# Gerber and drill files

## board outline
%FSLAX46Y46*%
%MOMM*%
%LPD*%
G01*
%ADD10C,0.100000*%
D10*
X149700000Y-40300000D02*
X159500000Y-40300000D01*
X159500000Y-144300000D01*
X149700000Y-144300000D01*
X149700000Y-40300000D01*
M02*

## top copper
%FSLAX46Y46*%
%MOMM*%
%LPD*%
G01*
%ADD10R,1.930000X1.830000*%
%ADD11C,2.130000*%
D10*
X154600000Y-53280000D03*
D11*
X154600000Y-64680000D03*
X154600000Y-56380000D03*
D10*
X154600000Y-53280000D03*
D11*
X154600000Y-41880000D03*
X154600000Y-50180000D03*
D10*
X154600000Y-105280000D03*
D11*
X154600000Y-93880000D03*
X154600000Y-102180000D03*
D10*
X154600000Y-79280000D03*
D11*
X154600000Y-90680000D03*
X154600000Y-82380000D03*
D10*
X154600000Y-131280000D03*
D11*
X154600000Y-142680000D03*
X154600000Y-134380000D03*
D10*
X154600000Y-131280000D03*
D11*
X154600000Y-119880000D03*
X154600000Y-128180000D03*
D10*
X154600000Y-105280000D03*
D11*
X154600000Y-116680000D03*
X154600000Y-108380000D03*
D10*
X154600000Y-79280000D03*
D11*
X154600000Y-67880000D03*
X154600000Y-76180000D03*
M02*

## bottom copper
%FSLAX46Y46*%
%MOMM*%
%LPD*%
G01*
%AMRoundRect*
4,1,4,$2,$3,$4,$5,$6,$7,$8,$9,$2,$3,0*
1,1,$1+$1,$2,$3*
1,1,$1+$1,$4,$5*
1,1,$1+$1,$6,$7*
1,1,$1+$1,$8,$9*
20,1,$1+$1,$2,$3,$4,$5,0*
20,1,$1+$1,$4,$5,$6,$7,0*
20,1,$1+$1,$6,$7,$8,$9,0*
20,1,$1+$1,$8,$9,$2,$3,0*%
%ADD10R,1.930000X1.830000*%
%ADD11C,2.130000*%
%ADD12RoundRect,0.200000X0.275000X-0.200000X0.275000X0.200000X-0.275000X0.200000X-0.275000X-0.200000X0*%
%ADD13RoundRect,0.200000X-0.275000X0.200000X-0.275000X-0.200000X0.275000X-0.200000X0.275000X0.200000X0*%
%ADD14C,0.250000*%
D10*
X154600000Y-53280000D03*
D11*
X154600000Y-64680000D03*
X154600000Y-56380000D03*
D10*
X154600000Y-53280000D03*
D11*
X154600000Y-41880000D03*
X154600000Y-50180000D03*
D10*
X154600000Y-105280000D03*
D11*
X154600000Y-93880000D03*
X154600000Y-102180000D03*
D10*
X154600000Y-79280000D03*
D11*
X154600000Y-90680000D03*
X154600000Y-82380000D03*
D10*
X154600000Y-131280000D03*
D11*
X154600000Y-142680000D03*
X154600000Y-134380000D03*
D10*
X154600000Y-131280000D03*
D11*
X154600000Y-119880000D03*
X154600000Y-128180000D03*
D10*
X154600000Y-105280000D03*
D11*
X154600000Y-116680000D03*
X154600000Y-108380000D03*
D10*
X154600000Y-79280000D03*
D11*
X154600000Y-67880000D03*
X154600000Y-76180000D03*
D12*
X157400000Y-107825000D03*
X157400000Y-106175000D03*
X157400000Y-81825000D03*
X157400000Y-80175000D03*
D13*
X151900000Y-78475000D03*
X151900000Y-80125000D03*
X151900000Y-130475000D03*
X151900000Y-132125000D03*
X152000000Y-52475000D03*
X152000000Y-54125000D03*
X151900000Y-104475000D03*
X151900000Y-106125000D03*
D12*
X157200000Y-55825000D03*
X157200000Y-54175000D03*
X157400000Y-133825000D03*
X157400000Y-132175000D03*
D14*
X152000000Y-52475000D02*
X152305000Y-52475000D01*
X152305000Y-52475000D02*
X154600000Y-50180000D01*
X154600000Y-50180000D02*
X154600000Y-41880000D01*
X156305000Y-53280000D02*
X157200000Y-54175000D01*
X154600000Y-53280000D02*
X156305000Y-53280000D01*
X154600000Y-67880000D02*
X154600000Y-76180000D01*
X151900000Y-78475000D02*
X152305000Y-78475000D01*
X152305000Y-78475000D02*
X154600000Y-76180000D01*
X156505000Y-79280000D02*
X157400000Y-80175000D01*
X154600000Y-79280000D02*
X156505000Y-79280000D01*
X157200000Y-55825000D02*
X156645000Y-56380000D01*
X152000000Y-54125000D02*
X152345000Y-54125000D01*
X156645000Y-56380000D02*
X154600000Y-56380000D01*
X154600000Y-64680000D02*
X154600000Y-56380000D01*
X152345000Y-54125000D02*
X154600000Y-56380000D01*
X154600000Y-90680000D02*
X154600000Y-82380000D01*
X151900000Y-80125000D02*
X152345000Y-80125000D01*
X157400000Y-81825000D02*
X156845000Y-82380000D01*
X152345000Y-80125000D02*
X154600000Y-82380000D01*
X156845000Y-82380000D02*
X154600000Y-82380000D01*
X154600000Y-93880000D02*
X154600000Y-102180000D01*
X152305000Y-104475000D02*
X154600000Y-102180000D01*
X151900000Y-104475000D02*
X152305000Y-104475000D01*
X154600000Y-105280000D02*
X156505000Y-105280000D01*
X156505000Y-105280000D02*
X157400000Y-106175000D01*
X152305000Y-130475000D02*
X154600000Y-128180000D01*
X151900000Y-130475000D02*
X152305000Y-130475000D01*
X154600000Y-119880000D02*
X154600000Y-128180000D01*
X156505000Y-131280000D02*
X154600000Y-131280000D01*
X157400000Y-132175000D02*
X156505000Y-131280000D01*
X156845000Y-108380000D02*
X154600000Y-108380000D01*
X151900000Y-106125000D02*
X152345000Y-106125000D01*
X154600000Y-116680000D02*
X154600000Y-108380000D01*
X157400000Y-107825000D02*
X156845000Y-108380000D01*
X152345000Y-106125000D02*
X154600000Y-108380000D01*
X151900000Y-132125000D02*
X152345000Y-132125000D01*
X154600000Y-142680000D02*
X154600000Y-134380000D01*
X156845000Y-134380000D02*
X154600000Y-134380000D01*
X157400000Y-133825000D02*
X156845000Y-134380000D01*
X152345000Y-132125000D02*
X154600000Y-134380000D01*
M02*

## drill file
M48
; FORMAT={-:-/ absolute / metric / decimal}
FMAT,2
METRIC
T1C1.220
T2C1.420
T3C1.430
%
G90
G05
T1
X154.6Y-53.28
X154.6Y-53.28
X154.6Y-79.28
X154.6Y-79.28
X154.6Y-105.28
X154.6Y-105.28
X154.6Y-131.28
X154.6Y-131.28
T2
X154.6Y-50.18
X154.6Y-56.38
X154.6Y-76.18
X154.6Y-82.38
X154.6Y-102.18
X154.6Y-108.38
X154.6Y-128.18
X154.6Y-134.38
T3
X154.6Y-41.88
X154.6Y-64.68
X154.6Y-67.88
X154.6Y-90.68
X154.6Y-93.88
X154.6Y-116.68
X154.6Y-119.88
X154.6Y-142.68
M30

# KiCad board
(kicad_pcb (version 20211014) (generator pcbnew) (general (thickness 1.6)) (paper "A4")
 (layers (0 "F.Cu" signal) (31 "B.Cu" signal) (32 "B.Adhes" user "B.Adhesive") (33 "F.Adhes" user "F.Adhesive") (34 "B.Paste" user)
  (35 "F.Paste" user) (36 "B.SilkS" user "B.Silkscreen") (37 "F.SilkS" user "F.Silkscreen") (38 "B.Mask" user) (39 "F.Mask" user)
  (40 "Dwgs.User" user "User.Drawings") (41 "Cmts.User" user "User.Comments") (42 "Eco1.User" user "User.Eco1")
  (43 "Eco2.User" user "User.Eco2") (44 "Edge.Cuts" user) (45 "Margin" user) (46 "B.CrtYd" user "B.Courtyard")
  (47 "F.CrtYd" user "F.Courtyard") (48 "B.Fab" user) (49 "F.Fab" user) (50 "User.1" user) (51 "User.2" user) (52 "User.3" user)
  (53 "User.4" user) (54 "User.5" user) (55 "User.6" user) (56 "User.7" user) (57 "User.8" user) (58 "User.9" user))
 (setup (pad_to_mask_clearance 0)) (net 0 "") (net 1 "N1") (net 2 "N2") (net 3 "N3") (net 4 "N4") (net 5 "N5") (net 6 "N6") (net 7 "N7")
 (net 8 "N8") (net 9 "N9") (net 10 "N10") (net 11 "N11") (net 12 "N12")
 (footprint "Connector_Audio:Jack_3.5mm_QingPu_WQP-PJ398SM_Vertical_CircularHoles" (layer "F.Cu") (at 154.6 53.28)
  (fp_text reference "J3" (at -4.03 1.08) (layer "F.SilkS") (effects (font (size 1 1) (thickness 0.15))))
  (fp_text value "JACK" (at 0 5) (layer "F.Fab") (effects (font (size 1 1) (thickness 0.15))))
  (pad "S" thru_hole rect locked (at 0 0 180) (size 1.93 1.83) (drill 1.22) (layers *.Cu *.Mask) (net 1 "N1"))
  (pad "T" thru_hole circle locked (at 0 11.4 180) (size 2.13 2.13) (drill 1.43) (layers *.Cu *.Mask) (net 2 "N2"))
  (pad "TN" thru_hole circle locked (at 0 3.1 180) (size 2.13 2.13) (drill 1.42) (layers *.Cu *.Mask) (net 2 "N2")))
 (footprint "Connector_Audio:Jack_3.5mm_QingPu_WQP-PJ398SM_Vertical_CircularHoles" (layer "F.Cu") (at 154.6 53.28 180)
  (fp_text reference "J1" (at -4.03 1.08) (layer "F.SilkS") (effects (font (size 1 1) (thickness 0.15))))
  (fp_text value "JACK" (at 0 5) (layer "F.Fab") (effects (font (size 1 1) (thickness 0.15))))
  (pad "S" thru_hole rect locked (at 0 0) (size 1.93 1.83) (drill 1.22) (layers *.Cu *.Mask) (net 1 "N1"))
  (pad "T" thru_hole circle locked (at 0 11.4) (size 2.13 2.13) (drill 1.43) (layers *.Cu *.Mask) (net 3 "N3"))
  (pad "TN" thru_hole circle locked (at 0 3.1) (size 2.13 2.13) (drill 1.42) (layers *.Cu *.Mask) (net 3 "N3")))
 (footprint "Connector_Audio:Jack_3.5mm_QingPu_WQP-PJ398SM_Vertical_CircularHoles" (layer "F.Cu") (at 154.6 105.28 180)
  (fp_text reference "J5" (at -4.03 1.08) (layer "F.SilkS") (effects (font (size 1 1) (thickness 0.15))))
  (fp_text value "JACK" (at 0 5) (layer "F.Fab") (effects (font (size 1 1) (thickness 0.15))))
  (pad "S" thru_hole rect locked (at 0 0) (size 1.93 1.83) (drill 1.22) (layers *.Cu *.Mask) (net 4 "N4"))
  (pad "T" thru_hole circle locked (at 0 11.4) (size 2.13 2.13) (drill 1.43) (layers *.Cu *.Mask) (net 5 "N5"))
  (pad "TN" thru_hole circle locked (at 0 3.1) (size 2.13 2.13) (drill 1.42) (layers *.Cu *.Mask) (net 5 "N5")))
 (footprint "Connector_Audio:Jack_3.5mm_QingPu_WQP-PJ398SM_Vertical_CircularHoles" (layer "F.Cu") (at 154.6 79.28)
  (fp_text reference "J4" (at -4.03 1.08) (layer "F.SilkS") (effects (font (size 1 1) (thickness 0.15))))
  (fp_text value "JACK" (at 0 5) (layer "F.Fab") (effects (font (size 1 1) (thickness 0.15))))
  (pad "S" thru_hole rect locked (at 0 0 180) (size 1.93 1.83) (drill 1.22) (layers *.Cu *.Mask) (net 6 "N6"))
  (pad "T" thru_hole circle locked (at 0 11.4 180) (size 2.13 2.13) (drill 1.43) (layers *.Cu *.Mask) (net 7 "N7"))
  (pad "TN" thru_hole circle locked (at 0 3.1 180) (size 2.13 2.13) (drill 1.42) (layers *.Cu *.Mask) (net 7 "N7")))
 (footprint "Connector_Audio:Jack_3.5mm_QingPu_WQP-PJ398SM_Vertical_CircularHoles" (layer "F.Cu") (at 154.6 131.28)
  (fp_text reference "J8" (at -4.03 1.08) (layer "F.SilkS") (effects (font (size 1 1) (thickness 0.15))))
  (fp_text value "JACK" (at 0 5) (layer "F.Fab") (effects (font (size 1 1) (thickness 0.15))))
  (pad "S" thru_hole rect locked (at 0 0 180) (size 1.93 1.83) (drill 1.22) (layers *.Cu *.Mask) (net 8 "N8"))
  (pad "T" thru_hole circle locked (at 0 11.4 180) (size 2.13 2.13) (drill 1.43) (layers *.Cu *.Mask) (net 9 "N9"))
  (pad "TN" thru_hole circle locked (at 0 3.1 180) (size 2.13 2.13) (drill 1.42) (layers *.Cu *.Mask) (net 9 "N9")))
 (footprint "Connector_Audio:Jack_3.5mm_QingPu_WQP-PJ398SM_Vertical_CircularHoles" (layer "F.Cu") (at 154.6 131.28 180)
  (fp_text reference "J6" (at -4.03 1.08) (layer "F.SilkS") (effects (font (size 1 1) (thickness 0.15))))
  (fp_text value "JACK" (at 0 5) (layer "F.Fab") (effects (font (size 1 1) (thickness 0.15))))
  (pad "S" thru_hole rect locked (at 0 0) (size 1.93 1.83) (drill 1.22) (layers *.Cu *.Mask) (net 8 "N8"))
  (pad "T" thru_hole circle locked (at 0 11.4) (size 2.13 2.13) (drill 1.43) (layers *.Cu *.Mask) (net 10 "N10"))
  (pad "TN" thru_hole circle locked (at 0 3.1) (size 2.13 2.13) (drill 1.42) (layers *.Cu *.Mask) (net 10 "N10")))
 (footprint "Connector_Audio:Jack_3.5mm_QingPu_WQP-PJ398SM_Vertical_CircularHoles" (layer "F.Cu") (at 154.6 105.28)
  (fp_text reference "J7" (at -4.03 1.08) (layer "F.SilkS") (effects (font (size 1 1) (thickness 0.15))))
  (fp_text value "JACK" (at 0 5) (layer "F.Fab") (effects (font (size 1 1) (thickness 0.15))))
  (pad "S" thru_hole rect locked (at 0 0 180) (size 1.93 1.83) (drill 1.22) (layers *.Cu *.Mask) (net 4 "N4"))
  (pad "T" thru_hole circle locked (at 0 11.4 180) (size 2.13 2.13) (drill 1.43) (layers *.Cu *.Mask) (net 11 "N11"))
  (pad "TN" thru_hole circle locked (at 0 3.1 180) (size 2.13 2.13) (drill 1.42) (layers *.Cu *.Mask) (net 11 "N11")))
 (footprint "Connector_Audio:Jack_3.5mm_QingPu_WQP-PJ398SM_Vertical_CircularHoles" (layer "F.Cu") (at 154.6 79.28 180)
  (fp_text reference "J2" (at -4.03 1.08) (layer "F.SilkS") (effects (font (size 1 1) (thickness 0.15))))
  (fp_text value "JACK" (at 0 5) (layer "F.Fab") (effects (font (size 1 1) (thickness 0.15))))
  (pad "S" thru_hole rect locked (at 0 0) (size 1.93 1.83) (drill 1.22) (layers *.Cu *.Mask) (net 6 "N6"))
  (pad "T" thru_hole circle locked (at 0 11.4) (size 2.13 2.13) (drill 1.43) (layers *.Cu *.Mask) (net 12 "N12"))
  (pad "TN" thru_hole circle locked (at 0 3.1) (size 2.13 2.13) (drill 1.42) (layers *.Cu *.Mask) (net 12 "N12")))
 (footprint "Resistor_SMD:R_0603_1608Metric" (layer "B.Cu") (at 157.4 107 90)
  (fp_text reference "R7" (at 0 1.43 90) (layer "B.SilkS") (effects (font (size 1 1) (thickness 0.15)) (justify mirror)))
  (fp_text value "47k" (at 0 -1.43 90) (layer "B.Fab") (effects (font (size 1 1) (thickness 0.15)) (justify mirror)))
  (pad "1" smd roundrect locked (at -0.825 0 90) (size 0.8 0.95) (layers "B.Cu" "B.Paste" "B.Mask") (roundrect_rratio 0.25) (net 11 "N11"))
  (pad "2" smd roundrect locked (at 0.825 0 90) (size 0.8 0.95) (layers "B.Cu" "B.Paste" "B.Mask") (roundrect_rratio 0.25) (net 4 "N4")))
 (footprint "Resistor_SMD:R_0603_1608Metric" (layer "B.Cu") (at 157.4 81 90)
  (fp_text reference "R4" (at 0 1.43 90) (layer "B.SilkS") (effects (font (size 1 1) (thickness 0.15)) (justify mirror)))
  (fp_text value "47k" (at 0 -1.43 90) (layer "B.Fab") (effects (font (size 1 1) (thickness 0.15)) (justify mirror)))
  (pad "1" smd roundrect locked (at -0.825 0 90) (size 0.8 0.95) (layers "B.Cu" "B.Paste" "B.Mask") (roundrect_rratio 0.25) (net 7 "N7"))
  (pad "2" smd roundrect locked (at 0.825 0 90) (size 0.8 0.95) (layers "B.Cu" "B.Paste" "B.Mask") (roundrect_rratio 0.25) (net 6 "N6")))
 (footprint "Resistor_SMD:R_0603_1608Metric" (layer "B.Cu") (at 151.9 79.3 -90)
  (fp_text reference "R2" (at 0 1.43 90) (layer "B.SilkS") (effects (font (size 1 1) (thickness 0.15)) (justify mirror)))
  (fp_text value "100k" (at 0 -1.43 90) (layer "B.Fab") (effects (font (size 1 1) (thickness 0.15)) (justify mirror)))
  (pad "1" smd roundrect locked (at -0.825 0 270) (size 0.8 0.95) (layers "B.Cu" "B.Paste" "B.Mask") (roundrect_rratio 0.25) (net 12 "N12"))
  (pad "2" smd roundrect locked (at 0.825 0 270) (size 0.8 0.95) (layers "B.Cu" "B.Paste" "B.Mask") (roundrect_rratio 0.25) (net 7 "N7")))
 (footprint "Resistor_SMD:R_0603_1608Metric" (layer "B.Cu") (at 151.9 131.3 -90)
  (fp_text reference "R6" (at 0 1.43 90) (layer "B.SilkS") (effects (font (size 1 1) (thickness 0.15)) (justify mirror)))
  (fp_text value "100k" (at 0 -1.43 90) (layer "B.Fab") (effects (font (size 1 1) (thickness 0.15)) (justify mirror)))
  (pad "1" smd roundrect locked (at -0.825 0 270) (size 0.8 0.95) (layers "B.Cu" "B.Paste" "B.Mask") (roundrect_rratio 0.25) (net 10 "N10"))
  (pad "2" smd roundrect locked (at 0.825 0 270) (size 0.8 0.95) (layers "B.Cu" "B.Paste" "B.Mask") (roundrect_rratio 0.25) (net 9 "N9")))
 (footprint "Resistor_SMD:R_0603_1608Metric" (layer "B.Cu") (at 152 53.3 -90)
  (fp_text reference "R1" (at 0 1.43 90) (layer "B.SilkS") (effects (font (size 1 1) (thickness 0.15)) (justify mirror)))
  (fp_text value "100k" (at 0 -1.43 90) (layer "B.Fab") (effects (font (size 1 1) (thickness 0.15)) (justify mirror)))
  (pad "1" smd roundrect locked (at -0.825 0 270) (size 0.8 0.95) (layers "B.Cu" "B.Paste" "B.Mask") (roundrect_rratio 0.25) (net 3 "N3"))
  (pad "2" smd roundrect locked (at 0.825 0 270) (size 0.8 0.95) (layers "B.Cu" "B.Paste" "B.Mask") (roundrect_rratio 0.25) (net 2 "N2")))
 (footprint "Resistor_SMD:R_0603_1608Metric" (layer "B.Cu") (at 151.9 105.3 -90)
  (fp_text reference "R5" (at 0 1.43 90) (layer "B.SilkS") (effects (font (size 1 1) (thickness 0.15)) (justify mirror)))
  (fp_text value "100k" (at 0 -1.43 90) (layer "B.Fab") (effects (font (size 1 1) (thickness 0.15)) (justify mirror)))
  (pad "1" smd roundrect locked (at -0.825 0 270) (size 0.8 0.95) (layers "B.Cu" "B.Paste" "B.Mask") (roundrect_rratio 0.25) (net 5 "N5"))
  (pad "2" smd roundrect locked (at 0.825 0 270) (size 0.8 0.95) (layers "B.Cu" "B.Paste" "B.Mask") (roundrect_rratio 0.25) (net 11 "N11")))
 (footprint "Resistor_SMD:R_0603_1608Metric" (layer "B.Cu") (at 157.2 55 90)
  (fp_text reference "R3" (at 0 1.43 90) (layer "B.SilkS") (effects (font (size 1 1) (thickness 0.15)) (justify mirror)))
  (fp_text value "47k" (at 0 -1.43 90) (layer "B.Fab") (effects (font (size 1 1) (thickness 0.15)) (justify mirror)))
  (pad "1" smd roundrect locked (at -0.825 0 90) (size 0.8 0.95) (layers "B.Cu" "B.Paste" "B.Mask") (roundrect_rratio 0.25) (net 2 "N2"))
  (pad "2" smd roundrect locked (at 0.825 0 90) (size 0.8 0.95) (layers "B.Cu" "B.Paste" "B.Mask") (roundrect_rratio 0.25) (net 1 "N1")))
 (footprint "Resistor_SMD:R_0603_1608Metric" (layer "B.Cu") (at 157.4 133 90)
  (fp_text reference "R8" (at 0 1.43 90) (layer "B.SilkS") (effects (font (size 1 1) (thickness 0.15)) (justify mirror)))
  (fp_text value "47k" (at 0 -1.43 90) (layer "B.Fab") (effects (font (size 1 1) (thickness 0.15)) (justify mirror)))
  (pad "1" smd roundrect locked (at -0.825 0 90) (size 0.8 0.95) (layers "B.Cu" "B.Paste" "B.Mask") (roundrect_rratio 0.25) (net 9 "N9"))
  (pad "2" smd roundrect locked (at 0.825 0 90) (size 0.8 0.95) (layers "B.Cu" "B.Paste" "B.Mask") (roundrect_rratio 0.25) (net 8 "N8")))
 (gr_rect (start 149.7 40.3) (end 159.5 144.3) (layer "Edge.Cuts") (width 0.1) (fill none))
 (segment (start 152 52.475) (end 152.305 52.475) (width 0.25) (layer "B.Cu") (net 3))
 (segment (start 152.305 52.475) (end 154.6 50.18) (width 0.25) (layer "B.Cu") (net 3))
 (segment (start 154.6 50.18) (end 154.6 41.88) (width 0.25) (layer "B.Cu") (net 3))
 (segment (start 156.305 53.28) (end 157.2 54.175) (width 0.25) (layer "B.Cu") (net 1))
 (segment (start 154.6 53.28) (end 156.305 53.28) (width 0.25) (layer "B.Cu") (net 1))
 (segment (start 154.6 67.88) (end 154.6 76.18) (width 0.25) (layer "B.Cu") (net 12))
 (segment (start 151.9 78.475) (end 152.305 78.475) (width 0.25) (layer "B.Cu") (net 12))
 (segment (start 152.305 78.475) (end 154.6 76.18) (width 0.25) (layer "B.Cu") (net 12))
 (segment (start 156.505 79.28) (end 157.4 80.175) (width 0.25) (layer "B.Cu") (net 6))
 (segment (start 154.6 79.28) (end 156.505 79.28) (width 0.25) (layer "B.Cu") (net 6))
 (segment (start 157.2 55.825) (end 156.645 56.38) (width 0.25) (layer "B.Cu") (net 2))
 (segment (start 152 54.125) (end 152.345 54.125) (width 0.25) (layer "B.Cu") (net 2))
 (segment (start 156.645 56.38) (end 154.6 56.38) (width 0.25) (layer "B.Cu") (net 2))
 (segment (start 154.6 64.68) (end 154.6 56.38) (width 0.25) (layer "B.Cu") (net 2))
 (segment (start 152.345 54.125) (end 154.6 56.38) (width 0.25) (layer "B.Cu") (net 2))
 (segment (start 154.6 90.68) (end 154.6 82.38) (width 0.25) (layer "B.Cu") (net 7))
 (segment (start 151.9 80.125) (end 152.345 80.125) (width 0.25) (layer "B.Cu") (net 7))
 (segment (start 157.4 81.825) (end 156.845 82.38) (width 0.25) (layer "B.Cu") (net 7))
 (segment (start 152.345 80.125) (end 154.6 82.38) (width 0.25) (layer "B.Cu") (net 7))
 (segment (start 156.845 82.38) (end 154.6 82.38) (width 0.25) (layer "B.Cu") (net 7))
 (segment (start 154.6 93.88) (end 154.6 102.18) (width 0.25) (layer "B.Cu") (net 5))
 (segment (start 152.305 104.475) (end 154.6 102.18) (width 0.25) (layer "B.Cu") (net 5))
 (segment (start 151.9 104.475) (end 152.305 104.475) (width 0.25) (layer "B.Cu") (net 5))
 (segment (start 154.6 105.28) (end 156.505 105.28) (width 0.25) (layer "B.Cu") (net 4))
 (segment (start 156.505 105.28) (end 157.4 106.175) (width 0.25) (layer "B.Cu") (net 4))
 (segment (start 152.305 130.475) (end 154.6 128.18) (width 0.25) (layer "B.Cu") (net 10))
 (segment (start 151.9 130.475) (end 152.305 130.475) (width 0.25) (layer "B.Cu") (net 10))
 (segment (start 154.6 119.88) (end 154.6 128.18) (width 0.25) (layer "B.Cu") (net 10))
 (segment (start 156.505 131.28) (end 154.6 131.28) (width 0.25) (layer "B.Cu") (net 8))
 (segment (start 157.4 132.175) (end 156.505 131.28) (width 0.25) (layer "B.Cu") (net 8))
 (segment (start 156.845 108.38) (end 154.6 108.38) (width 0.25) (layer "B.Cu") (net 11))
 (segment (start 151.9 106.125) (end 152.345 106.125) (width 0.25) (layer "B.Cu") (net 11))
 (segment (start 154.6 116.68) (end 154.6 108.38) (width 0.25) (layer "B.Cu") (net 11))
 (segment (start 157.4 107.825) (end 156.845 108.38) (width 0.25) (layer "B.Cu") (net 11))
 (segment (start 152.345 106.125) (end 154.6 108.38) (width 0.25) (layer "B.Cu") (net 11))
 (segment (start 151.9 132.125) (end 152.345 132.125) (width 0.25) (layer "B.Cu") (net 9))
 (segment (start 154.6 142.68) (end 154.6 134.38) (width 0.25) (layer "B.Cu") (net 9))
 (segment (start 156.845 134.38) (end 154.6 134.38) (width 0.25) (layer "B.Cu") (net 9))
 (segment (start 157.4 133.825) (end 156.845 134.38) (width 0.25) (layer "B.Cu") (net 9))
 (segment (start 152.345 132.125) (end 154.6 134.38) (width 0.25) (layer "B.Cu") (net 9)))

